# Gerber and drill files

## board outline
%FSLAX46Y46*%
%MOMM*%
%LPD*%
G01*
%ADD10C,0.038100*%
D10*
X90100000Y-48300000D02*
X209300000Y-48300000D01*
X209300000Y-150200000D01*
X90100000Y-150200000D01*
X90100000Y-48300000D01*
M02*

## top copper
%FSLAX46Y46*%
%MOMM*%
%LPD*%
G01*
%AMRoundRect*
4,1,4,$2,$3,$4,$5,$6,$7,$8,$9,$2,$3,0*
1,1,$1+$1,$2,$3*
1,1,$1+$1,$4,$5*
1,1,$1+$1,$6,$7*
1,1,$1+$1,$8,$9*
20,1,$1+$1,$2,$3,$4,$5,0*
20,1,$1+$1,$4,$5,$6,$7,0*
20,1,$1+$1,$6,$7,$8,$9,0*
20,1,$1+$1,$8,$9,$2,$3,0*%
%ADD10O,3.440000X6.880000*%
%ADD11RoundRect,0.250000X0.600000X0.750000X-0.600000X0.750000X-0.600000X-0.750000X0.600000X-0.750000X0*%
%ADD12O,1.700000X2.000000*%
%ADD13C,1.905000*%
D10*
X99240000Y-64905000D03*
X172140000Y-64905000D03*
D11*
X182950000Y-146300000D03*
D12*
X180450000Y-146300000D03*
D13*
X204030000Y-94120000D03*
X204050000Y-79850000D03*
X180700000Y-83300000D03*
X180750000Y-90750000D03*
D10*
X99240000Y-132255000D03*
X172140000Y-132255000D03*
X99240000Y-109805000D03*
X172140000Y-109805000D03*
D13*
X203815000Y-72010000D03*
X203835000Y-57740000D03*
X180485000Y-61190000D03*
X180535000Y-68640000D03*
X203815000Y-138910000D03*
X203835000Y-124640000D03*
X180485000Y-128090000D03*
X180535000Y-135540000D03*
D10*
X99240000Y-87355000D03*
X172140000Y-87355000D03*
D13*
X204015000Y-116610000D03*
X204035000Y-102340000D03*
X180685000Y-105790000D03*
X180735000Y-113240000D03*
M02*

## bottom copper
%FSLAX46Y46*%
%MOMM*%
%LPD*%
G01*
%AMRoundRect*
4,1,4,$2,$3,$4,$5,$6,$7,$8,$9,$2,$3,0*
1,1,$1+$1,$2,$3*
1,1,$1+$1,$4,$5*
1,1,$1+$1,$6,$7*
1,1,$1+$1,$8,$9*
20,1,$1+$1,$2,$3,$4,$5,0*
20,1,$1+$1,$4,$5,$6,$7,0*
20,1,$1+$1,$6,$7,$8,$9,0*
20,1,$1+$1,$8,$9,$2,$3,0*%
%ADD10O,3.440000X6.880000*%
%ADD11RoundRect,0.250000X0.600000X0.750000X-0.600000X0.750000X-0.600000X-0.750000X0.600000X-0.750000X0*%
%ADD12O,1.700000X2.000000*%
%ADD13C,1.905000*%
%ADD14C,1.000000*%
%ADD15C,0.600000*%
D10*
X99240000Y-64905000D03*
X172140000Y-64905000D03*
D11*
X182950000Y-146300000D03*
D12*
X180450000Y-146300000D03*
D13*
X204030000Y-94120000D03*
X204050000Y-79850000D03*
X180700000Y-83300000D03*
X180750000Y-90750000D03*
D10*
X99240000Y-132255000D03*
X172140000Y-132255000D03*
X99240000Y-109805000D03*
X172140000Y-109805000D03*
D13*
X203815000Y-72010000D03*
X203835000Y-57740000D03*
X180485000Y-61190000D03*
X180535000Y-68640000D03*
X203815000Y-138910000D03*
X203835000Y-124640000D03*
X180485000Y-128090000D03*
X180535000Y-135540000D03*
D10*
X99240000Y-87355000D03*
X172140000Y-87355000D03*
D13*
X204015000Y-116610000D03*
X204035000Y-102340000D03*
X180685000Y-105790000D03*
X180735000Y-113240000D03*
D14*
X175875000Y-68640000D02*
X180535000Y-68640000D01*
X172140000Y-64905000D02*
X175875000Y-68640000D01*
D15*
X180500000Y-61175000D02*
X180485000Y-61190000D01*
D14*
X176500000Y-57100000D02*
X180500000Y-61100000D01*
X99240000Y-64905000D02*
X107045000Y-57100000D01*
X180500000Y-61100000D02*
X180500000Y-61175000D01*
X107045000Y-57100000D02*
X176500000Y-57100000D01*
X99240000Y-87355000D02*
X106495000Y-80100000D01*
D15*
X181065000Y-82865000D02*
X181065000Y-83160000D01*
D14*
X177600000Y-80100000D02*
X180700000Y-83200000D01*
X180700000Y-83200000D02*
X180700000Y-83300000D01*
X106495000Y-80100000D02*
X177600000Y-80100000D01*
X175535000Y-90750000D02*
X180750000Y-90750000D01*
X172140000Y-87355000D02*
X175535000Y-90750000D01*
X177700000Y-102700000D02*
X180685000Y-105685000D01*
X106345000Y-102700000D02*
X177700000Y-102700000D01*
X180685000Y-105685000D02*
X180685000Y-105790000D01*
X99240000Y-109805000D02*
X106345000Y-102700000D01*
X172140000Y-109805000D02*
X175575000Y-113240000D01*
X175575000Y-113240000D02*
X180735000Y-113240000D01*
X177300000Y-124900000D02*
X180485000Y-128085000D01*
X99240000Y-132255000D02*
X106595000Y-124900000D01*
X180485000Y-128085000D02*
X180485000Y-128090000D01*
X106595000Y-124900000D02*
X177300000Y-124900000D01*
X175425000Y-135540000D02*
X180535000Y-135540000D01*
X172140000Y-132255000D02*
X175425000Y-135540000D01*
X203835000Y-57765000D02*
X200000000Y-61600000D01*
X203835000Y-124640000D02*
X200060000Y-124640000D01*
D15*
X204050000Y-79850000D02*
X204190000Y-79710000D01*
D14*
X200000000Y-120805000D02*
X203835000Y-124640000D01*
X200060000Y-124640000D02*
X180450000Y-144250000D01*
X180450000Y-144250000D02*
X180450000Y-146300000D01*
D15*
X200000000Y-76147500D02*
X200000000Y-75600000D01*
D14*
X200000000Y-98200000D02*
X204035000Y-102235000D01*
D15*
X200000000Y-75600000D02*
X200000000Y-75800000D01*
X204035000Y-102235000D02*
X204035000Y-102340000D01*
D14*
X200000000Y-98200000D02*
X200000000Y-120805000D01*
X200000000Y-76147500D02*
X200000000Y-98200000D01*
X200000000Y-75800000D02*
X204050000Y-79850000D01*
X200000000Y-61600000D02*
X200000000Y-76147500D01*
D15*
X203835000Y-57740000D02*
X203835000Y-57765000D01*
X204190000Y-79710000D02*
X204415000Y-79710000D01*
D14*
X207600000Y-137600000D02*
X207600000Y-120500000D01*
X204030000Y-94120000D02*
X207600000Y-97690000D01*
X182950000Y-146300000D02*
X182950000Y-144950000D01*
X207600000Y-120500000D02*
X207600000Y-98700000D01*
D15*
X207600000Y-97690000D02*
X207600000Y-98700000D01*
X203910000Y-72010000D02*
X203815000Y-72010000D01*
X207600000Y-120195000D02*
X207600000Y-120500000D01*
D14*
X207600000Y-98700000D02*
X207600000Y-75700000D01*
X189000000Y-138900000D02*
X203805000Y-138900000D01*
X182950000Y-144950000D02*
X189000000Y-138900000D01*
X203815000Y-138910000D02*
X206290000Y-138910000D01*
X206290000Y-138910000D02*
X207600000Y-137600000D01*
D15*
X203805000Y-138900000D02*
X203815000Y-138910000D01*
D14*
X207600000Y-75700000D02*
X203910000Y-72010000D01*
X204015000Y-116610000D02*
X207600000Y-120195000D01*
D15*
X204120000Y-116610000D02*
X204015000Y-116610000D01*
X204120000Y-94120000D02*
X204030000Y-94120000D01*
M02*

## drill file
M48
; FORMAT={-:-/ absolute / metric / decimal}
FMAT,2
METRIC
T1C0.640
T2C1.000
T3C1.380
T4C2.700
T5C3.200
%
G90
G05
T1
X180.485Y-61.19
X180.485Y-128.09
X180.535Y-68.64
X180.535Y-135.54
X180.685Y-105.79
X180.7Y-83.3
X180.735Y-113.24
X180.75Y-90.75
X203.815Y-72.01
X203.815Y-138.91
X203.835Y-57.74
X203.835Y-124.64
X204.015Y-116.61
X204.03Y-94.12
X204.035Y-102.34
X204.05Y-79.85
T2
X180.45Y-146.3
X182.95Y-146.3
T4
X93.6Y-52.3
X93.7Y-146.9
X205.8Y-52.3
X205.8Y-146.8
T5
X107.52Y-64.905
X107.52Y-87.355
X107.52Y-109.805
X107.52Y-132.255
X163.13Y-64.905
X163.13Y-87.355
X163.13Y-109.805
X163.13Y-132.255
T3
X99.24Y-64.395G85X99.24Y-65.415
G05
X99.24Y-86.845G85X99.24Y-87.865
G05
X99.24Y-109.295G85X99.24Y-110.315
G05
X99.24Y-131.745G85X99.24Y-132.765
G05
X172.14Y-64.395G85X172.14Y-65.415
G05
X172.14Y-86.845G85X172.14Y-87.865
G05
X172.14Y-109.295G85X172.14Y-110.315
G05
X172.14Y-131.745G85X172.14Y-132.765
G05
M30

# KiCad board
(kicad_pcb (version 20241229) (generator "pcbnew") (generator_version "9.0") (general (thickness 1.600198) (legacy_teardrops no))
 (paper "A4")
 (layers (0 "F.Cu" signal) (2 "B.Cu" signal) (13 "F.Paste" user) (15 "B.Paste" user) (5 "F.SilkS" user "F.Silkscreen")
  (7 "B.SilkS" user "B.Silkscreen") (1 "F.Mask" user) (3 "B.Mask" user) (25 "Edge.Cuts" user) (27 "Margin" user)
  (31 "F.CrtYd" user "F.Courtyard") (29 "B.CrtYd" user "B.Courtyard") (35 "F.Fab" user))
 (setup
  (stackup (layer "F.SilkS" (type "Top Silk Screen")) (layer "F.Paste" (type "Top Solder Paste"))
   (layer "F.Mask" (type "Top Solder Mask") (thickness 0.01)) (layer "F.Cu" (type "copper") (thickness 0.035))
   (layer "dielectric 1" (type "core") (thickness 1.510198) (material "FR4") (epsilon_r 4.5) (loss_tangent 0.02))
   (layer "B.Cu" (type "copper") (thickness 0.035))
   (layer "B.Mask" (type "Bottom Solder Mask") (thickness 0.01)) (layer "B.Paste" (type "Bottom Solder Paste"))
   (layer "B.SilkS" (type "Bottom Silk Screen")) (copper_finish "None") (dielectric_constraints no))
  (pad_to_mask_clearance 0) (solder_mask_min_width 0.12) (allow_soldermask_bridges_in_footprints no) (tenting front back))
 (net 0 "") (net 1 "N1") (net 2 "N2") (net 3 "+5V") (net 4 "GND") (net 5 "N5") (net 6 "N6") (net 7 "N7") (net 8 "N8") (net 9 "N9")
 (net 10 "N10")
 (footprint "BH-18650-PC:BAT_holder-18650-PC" (layer "F.Cu") (at 135.69 64.905)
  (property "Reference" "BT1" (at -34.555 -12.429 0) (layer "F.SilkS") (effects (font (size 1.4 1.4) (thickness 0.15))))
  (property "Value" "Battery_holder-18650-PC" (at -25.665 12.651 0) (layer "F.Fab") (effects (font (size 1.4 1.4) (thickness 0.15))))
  (pad "" np_thru_hole circle (at -28.17 0) (size 3.2 3.2) (drill 3.2) (layers "*.Cu" "*.Mask"))
  (pad "" np_thru_hole circle (at 27.44 0) (size 3.2 3.2) (drill 3.2) (layers "*.Cu" "*.Mask"))
  (pad "N" thru_hole oval (at -36.45 0) (size 3.44 6.88) (drill oval 1.38 2.4) (layers "*.Cu" "*.Mask") (remove_unused_layers no)
   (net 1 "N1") (solder_mask_margin 0.102))
  (pad "P" thru_hole oval (at 36.45 0) (size 3.44 6.88) (drill oval 1.38 2.4) (layers "*.Cu" "*.Mask") (remove_unused_layers no)
   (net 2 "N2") (solder_mask_margin 0.102)))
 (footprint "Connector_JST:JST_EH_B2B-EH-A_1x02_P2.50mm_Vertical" (layer "F.Cu") (at 182.95 146.3 180)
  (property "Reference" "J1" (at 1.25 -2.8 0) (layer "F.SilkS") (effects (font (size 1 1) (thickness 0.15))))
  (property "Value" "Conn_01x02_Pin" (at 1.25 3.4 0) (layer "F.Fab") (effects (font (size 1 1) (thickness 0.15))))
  (pad "1" thru_hole roundrect (at 0 0 180) (size 1.7 2) (drill 1) (layers "*.Cu" "*.Mask") (remove_unused_layers no)
   (roundrect_rratio 0.147059) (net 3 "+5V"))
  (pad "2" thru_hole oval (at 2.5 0 180) (size 1.7 2) (drill 1) (layers "*.Cu" "*.Mask") (remove_unused_layers no) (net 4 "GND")))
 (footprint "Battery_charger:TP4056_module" (layer "F.Cu") (at 206.55 78.5 180)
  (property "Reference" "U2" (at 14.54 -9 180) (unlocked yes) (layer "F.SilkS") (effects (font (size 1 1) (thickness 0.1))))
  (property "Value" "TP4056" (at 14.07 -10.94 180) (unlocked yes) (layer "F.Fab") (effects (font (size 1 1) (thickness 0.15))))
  (pad "1" thru_hole circle (at 2.52 -15.62 180) (size 1.905 1.905) (drill 0.64) (layers "*.Cu" "*.Mask") (remove_unused_layers no)
   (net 3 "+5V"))
  (pad "2" thru_hole circle (at 2.5 -1.35 180) (size 1.905 1.905) (drill 0.64) (layers "*.Cu" "*.Mask") (remove_unused_layers no)
   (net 4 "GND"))
  (pad "3" thru_hole circle (at 25.85 -4.8 180) (size 1.905 1.905) (drill 0.64) (layers "*.Cu" "*.Mask") (remove_unused_layers no)
   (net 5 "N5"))
  (pad "4" thru_hole circle (at 25.8 -12.25 180) (size 1.905 1.905) (drill 0.64) (layers "*.Cu" "*.Mask") (remove_unused_layers no)
   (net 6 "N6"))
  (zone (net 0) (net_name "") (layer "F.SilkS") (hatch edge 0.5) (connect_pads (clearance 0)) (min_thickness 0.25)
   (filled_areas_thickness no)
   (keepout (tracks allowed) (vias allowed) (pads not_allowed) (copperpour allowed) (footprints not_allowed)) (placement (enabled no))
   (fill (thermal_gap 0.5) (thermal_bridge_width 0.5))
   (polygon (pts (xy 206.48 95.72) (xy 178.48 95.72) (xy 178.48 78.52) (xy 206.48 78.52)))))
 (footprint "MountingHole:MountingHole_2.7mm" (layer "F.Cu") (at 205.8 146.8)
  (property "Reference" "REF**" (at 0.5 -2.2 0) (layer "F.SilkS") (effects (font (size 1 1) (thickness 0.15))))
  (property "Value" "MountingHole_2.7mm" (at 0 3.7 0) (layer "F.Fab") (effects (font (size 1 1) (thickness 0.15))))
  (pad "" np_thru_hole circle (at 0 0) (size 2.7 2.7) (drill 2.7) (layers "*.Cu" "*.Mask")))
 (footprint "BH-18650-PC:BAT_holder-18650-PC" (layer "F.Cu") (at 135.69 132.255)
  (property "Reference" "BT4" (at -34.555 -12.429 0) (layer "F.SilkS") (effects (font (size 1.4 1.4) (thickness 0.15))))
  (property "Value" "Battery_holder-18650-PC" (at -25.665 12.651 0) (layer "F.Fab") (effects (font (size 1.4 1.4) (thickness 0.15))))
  (pad "" np_thru_hole circle (at -28.17 0) (size 3.2 3.2) (drill 3.2) (layers "*.Cu" "*.Mask"))
  (pad "" np_thru_hole circle (at 27.44 0) (size 3.2 3.2) (drill 3.2) (layers "*.Cu" "*.Mask"))
  (pad "N" thru_hole oval (at -36.45 0) (size 3.44 6.88) (drill oval 1.38 2.4) (layers "*.Cu" "*.Mask") (remove_unused_layers no)
   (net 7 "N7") (solder_mask_margin 0.102))
  (pad "P" thru_hole oval (at 36.45 0) (size 3.44 6.88) (drill oval 1.38 2.4) (layers "*.Cu" "*.Mask") (remove_unused_layers no)
   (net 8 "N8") (solder_mask_margin 0.102)))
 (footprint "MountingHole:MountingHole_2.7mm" (layer "F.Cu") (at 93.6 52.3)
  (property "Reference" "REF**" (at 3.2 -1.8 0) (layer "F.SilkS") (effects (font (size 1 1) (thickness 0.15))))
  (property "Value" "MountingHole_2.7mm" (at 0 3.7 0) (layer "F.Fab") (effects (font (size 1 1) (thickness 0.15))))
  (pad "" np_thru_hole circle (at 0 0) (size 2.7 2.7) (drill 2.7) (layers "*.Cu" "*.Mask")))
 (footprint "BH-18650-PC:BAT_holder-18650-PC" (layer "F.Cu") (at 135.69 109.805)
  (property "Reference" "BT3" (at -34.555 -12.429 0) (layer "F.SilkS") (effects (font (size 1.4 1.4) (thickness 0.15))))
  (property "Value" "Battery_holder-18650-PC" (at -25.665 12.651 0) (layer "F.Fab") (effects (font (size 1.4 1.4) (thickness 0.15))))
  (pad "" np_thru_hole circle (at -28.17 0) (size 3.2 3.2) (drill 3.2) (layers "*.Cu" "*.Mask"))
  (pad "" np_thru_hole circle (at 27.44 0) (size 3.2 3.2) (drill 3.2) (layers "*.Cu" "*.Mask"))
  (pad "N" thru_hole oval (at -36.45 0) (size 3.44 6.88) (drill oval 1.38 2.4) (layers "*.Cu" "*.Mask") (remove_unused_layers no)
   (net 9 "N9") (solder_mask_margin 0.102))
  (pad "P" thru_hole oval (at 36.45 0) (size 3.44 6.88) (drill oval 1.38 2.4) (layers "*.Cu" "*.Mask") (remove_unused_layers no)
   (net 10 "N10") (solder_mask_margin 0.102)))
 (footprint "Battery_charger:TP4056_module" (layer "F.Cu") (at 206.335 56.39 180)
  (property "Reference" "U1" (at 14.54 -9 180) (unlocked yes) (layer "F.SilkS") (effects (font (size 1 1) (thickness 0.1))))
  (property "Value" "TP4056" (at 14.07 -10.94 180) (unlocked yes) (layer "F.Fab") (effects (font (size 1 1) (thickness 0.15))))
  (pad "1" thru_hole circle (at 2.52 -15.62 180) (size 1.905 1.905) (drill 0.64) (layers "*.Cu" "*.Mask") (remove_unused_layers no)
   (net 3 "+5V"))
  (pad "2" thru_hole circle (at 2.5 -1.35 180) (size 1.905 1.905) (drill 0.64) (layers "*.Cu" "*.Mask") (remove_unused_layers no)
   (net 4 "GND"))
  (pad "3" thru_hole circle (at 25.85 -4.8 180) (size 1.905 1.905) (drill 0.64) (layers "*.Cu" "*.Mask") (remove_unused_layers no)
   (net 1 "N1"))
  (pad "4" thru_hole circle (at 25.8 -12.25 180) (size 1.905 1.905) (drill 0.64) (layers "*.Cu" "*.Mask") (remove_unused_layers no)
   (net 2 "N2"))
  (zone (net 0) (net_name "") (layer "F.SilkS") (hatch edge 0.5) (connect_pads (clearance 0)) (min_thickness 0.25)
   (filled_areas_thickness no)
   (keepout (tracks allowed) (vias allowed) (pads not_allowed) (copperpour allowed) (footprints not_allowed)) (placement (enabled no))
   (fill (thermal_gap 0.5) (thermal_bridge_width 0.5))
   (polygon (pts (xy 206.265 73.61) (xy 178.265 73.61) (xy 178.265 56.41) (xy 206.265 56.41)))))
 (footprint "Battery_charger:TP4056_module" (layer "F.Cu") (at 206.335 123.29 180)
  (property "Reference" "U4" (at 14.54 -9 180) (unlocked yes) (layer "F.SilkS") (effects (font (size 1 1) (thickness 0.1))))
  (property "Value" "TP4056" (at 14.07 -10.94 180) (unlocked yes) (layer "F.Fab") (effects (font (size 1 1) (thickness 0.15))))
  (pad "1" thru_hole circle (at 2.52 -15.62 180) (size 1.905 1.905) (drill 0.64) (layers "*.Cu" "*.Mask") (remove_unused_layers no)
   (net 3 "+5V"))
  (pad "2" thru_hole circle (at 2.5 -1.35 180) (size 1.905 1.905) (drill 0.64) (layers "*.Cu" "*.Mask") (remove_unused_layers no)
   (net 4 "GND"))
  (pad "3" thru_hole circle (at 25.85 -4.8 180) (size 1.905 1.905) (drill 0.64) (layers "*.Cu" "*.Mask") (remove_unused_layers no)
   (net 7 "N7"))
  (pad "4" thru_hole circle (at 25.8 -12.25 180) (size 1.905 1.905) (drill 0.64) (layers "*.Cu" "*.Mask") (remove_unused_layers no)
   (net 8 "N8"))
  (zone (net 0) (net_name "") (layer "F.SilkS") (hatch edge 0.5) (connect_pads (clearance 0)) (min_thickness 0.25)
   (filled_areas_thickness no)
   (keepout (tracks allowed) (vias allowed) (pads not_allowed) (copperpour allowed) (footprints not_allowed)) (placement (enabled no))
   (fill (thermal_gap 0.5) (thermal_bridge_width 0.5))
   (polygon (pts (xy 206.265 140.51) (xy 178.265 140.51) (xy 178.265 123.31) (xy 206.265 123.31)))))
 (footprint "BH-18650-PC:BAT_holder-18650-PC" (layer "F.Cu") (at 135.69 87.355)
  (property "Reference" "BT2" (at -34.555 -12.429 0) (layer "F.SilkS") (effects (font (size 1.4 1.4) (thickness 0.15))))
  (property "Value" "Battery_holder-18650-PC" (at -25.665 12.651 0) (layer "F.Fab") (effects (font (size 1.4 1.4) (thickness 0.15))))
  (pad "" np_thru_hole circle (at -28.17 0) (size 3.2 3.2) (drill 3.2) (layers "*.Cu" "*.Mask"))
  (pad "" np_thru_hole circle (at 27.44 0) (size 3.2 3.2) (drill 3.2) (layers "*.Cu" "*.Mask"))
  (pad "N" thru_hole oval (at -36.45 0) (size 3.44 6.88) (drill oval 1.38 2.4) (layers "*.Cu" "*.Mask") (remove_unused_layers no)
   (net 5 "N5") (solder_mask_margin 0.102))
  (pad "P" thru_hole oval (at 36.45 0) (size 3.44 6.88) (drill oval 1.38 2.4) (layers "*.Cu" "*.Mask") (remove_unused_layers no)
   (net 6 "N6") (solder_mask_margin 0.102)))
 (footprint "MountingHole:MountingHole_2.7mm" (layer "F.Cu") (at 93.7 146.9)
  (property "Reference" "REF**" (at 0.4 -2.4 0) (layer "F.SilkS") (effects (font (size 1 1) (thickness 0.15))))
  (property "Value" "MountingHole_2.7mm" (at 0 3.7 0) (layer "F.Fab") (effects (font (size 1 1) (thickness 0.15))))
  (pad "" np_thru_hole circle (at 0 0) (size 2.7 2.7) (drill 2.7) (layers "*.Cu" "*.Mask")))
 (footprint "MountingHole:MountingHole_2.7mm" (layer "F.Cu") (at 205.8 52.3)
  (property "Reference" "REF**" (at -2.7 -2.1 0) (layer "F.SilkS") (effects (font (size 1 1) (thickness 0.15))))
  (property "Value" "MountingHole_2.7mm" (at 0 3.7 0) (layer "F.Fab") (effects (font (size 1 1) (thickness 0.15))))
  (pad "" np_thru_hole circle (at 0 0) (size 2.7 2.7) (drill 2.7) (layers "*.Cu" "*.Mask")))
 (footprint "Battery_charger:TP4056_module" (layer "F.Cu") (at 206.535 100.99 180)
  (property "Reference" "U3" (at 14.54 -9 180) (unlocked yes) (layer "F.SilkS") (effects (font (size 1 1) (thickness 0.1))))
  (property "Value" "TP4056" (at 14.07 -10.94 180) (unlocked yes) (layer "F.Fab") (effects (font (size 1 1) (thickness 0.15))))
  (pad "1" thru_hole circle (at 2.52 -15.62 180) (size 1.905 1.905) (drill 0.64) (layers "*.Cu" "*.Mask") (remove_unused_layers no)
   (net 3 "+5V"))
  (pad "2" thru_hole circle (at 2.5 -1.35 180) (size 1.905 1.905) (drill 0.64) (layers "*.Cu" "*.Mask") (remove_unused_layers no)
   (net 4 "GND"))
  (pad "3" thru_hole circle (at 25.85 -4.8 180) (size 1.905 1.905) (drill 0.64) (layers "*.Cu" "*.Mask") (remove_unused_layers no)
   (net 9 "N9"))
  (pad "4" thru_hole circle (at 25.8 -12.25 180) (size 1.905 1.905) (drill 0.64) (layers "*.Cu" "*.Mask") (remove_unused_layers no)
   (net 10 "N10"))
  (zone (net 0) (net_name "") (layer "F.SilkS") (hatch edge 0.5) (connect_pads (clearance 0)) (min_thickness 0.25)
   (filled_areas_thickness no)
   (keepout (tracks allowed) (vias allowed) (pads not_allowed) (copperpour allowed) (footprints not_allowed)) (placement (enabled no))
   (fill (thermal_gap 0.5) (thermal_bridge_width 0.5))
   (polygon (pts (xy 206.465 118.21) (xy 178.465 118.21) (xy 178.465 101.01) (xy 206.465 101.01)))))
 (gr_rect (start 90.1 48.3) (end 209.3 150.2) (stroke (width 0.0381) (type default)) (fill no) (layer "Edge.Cuts"))
 (segment (start 175.875 68.64) (end 180.535 68.64) (width 1) (layer "B.Cu") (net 2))
 (segment (start 172.14 64.905) (end 175.875 68.64) (width 1) (layer "B.Cu") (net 2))
 (segment (start 180.5 61.175) (end 180.485 61.19) (width 0.6) (layer "B.Cu") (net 1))
 (segment (start 176.5 57.1) (end 180.5 61.1) (width 1) (layer "B.Cu") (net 1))
 (segment (start 99.24 64.905) (end 107.045 57.1) (width 1) (layer "B.Cu") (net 1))
 (segment (start 180.5 61.1) (end 180.5 61.175) (width 1) (layer "B.Cu") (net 1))
 (segment (start 107.045 57.1) (end 176.5 57.1) (width 1) (layer "B.Cu") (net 1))
 (segment (start 99.24 87.355) (end 106.495 80.1) (width 1) (layer "B.Cu") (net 5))
 (segment (start 181.065 82.865) (end 181.065 83.16) (width 0.6) (layer "B.Cu") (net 5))
 (segment (start 177.6 80.1) (end 180.7 83.2) (width 1) (layer "B.Cu") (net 5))
 (segment (start 180.7 83.2) (end 180.7 83.3) (width 1) (layer "B.Cu") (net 5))
 (segment (start 106.495 80.1) (end 177.6 80.1) (width 1) (layer "B.Cu") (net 5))
 (segment (start 175.535 90.75) (end 180.75 90.75) (width 1) (layer "B.Cu") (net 6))
 (segment (start 172.14 87.355) (end 175.535 90.75) (width 1) (layer "B.Cu") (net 6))
 (segment (start 177.7 102.7) (end 180.685 105.685) (width 1) (layer "B.Cu") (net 9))
 (segment (start 106.345 102.7) (end 177.7 102.7) (width 1) (layer "B.Cu") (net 9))
 (segment (start 180.685 105.685) (end 180.685 105.79) (width 1) (layer "B.Cu") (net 9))
 (segment (start 99.24 109.805) (end 106.345 102.7) (width 1) (layer "B.Cu") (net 9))
 (segment (start 172.14 109.805) (end 175.575 113.24) (width 1) (layer "B.Cu") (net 10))
 (segment (start 175.575 113.24) (end 180.735 113.24) (width 1) (layer "B.Cu") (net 10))
 (segment (start 177.3 124.9) (end 180.485 128.085) (width 1) (layer "B.Cu") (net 7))
 (segment (start 99.24 132.255) (end 106.595 124.9) (width 1) (layer "B.Cu") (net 7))
 (segment (start 180.485 128.085) (end 180.485 128.09) (width 1) (layer "B.Cu") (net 7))
 (segment (start 106.595 124.9) (end 177.3 124.9) (width 1) (layer "B.Cu") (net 7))
 (segment (start 175.425 135.54) (end 180.535 135.54) (width 1) (layer "B.Cu") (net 8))
 (segment (start 172.14 132.255) (end 175.425 135.54) (width 1) (layer "B.Cu") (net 8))
 (segment (start 203.835 57.765) (end 200 61.6) (width 1) (layer "B.Cu") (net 4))
 (segment (start 203.835 124.64) (end 200.06 124.64) (width 1) (layer "B.Cu") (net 4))
 (segment (start 204.05 79.85) (end 204.19 79.71) (width 0.6) (layer "B.Cu") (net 4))
 (segment (start 200 120.805) (end 203.835 124.64) (width 1) (layer "B.Cu") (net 4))
 (segment (start 200.06 124.64) (end 180.45 144.25) (width 1) (layer "B.Cu") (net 4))
 (segment (start 180.45 144.25) (end 180.45 146.3) (width 1) (layer "B.Cu") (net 4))
 (segment (start 200 76.1475) (end 200 75.6) (width 0.6) (layer "B.Cu") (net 4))
 (segment (start 200 98.2) (end 204.035 102.235) (width 1) (layer "B.Cu") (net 4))
 (segment (start 200 75.6) (end 200 75.8) (width 0.6) (layer "B.Cu") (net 4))
 (segment (start 204.035 102.235) (end 204.035 102.34) (width 0.6) (layer "B.Cu") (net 4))
 (segment (start 200 98.2) (end 200 120.805) (width 1) (layer "B.Cu") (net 4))
 (segment (start 200 76.1475) (end 200 98.2) (width 1) (layer "B.Cu") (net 4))
 (segment (start 200 75.8) (end 204.05 79.85) (width 1) (layer "B.Cu") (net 4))
 (segment (start 200 61.6) (end 200 76.1475) (width 1) (layer "B.Cu") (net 4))
 (segment (start 203.835 57.74) (end 203.835 57.765) (width 0.6) (layer "B.Cu") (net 4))
 (segment (start 204.19 79.71) (end 204.415 79.71) (width 0.6) (layer "B.Cu") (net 4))
 (segment (start 207.6 137.6) (end 207.6 120.5) (width 1) (layer "B.Cu") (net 3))
 (segment (start 204.03 94.12) (end 207.6 97.69) (width 1) (layer "B.Cu") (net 3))
 (segment (start 182.95 146.3) (end 182.95 144.95) (width 1) (layer "B.Cu") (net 3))
 (segment (start 207.6 120.5) (end 207.6 98.7) (width 1) (layer "B.Cu") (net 3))
 (segment (start 207.6 97.69) (end 207.6 98.7) (width 0.6) (layer "B.Cu") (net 3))
 (segment (start 203.91 72.01) (end 203.815 72.01) (width 0.6) (layer "B.Cu") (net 3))
 (segment (start 207.6 120.195) (end 207.6 120.5) (width 0.6) (layer "B.Cu") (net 3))
 (segment (start 207.6 98.7) (end 207.6 75.7) (width 1) (layer "B.Cu") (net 3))
 (segment (start 189 138.9) (end 203.805 138.9) (width 1) (layer "B.Cu") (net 3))
 (segment (start 182.95 144.95) (end 189 138.9) (width 1) (layer "B.Cu") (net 3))
 (segment (start 203.815 138.91) (end 206.29 138.91) (width 1) (layer "B.Cu") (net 3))
 (segment (start 206.29 138.91) (end 207.6 137.6) (width 1) (layer "B.Cu") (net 3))
 (segment (start 203.805 138.9) (end 203.815 138.91) (width 0.6) (layer "B.Cu") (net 3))
 (segment (start 207.6 75.7) (end 203.91 72.01) (width 1) (layer "B.Cu") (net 3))
 (segment (start 204.015 116.61) (end 207.6 120.195) (width 1) (layer "B.Cu") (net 3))
 (segment (start 204.12 116.61) (end 204.015 116.61) (width 0.6) (layer "B.Cu") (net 3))
 (segment (start 204.12 94.12) (end 204.03 94.12) (width 0.6) (layer "B.Cu") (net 3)))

